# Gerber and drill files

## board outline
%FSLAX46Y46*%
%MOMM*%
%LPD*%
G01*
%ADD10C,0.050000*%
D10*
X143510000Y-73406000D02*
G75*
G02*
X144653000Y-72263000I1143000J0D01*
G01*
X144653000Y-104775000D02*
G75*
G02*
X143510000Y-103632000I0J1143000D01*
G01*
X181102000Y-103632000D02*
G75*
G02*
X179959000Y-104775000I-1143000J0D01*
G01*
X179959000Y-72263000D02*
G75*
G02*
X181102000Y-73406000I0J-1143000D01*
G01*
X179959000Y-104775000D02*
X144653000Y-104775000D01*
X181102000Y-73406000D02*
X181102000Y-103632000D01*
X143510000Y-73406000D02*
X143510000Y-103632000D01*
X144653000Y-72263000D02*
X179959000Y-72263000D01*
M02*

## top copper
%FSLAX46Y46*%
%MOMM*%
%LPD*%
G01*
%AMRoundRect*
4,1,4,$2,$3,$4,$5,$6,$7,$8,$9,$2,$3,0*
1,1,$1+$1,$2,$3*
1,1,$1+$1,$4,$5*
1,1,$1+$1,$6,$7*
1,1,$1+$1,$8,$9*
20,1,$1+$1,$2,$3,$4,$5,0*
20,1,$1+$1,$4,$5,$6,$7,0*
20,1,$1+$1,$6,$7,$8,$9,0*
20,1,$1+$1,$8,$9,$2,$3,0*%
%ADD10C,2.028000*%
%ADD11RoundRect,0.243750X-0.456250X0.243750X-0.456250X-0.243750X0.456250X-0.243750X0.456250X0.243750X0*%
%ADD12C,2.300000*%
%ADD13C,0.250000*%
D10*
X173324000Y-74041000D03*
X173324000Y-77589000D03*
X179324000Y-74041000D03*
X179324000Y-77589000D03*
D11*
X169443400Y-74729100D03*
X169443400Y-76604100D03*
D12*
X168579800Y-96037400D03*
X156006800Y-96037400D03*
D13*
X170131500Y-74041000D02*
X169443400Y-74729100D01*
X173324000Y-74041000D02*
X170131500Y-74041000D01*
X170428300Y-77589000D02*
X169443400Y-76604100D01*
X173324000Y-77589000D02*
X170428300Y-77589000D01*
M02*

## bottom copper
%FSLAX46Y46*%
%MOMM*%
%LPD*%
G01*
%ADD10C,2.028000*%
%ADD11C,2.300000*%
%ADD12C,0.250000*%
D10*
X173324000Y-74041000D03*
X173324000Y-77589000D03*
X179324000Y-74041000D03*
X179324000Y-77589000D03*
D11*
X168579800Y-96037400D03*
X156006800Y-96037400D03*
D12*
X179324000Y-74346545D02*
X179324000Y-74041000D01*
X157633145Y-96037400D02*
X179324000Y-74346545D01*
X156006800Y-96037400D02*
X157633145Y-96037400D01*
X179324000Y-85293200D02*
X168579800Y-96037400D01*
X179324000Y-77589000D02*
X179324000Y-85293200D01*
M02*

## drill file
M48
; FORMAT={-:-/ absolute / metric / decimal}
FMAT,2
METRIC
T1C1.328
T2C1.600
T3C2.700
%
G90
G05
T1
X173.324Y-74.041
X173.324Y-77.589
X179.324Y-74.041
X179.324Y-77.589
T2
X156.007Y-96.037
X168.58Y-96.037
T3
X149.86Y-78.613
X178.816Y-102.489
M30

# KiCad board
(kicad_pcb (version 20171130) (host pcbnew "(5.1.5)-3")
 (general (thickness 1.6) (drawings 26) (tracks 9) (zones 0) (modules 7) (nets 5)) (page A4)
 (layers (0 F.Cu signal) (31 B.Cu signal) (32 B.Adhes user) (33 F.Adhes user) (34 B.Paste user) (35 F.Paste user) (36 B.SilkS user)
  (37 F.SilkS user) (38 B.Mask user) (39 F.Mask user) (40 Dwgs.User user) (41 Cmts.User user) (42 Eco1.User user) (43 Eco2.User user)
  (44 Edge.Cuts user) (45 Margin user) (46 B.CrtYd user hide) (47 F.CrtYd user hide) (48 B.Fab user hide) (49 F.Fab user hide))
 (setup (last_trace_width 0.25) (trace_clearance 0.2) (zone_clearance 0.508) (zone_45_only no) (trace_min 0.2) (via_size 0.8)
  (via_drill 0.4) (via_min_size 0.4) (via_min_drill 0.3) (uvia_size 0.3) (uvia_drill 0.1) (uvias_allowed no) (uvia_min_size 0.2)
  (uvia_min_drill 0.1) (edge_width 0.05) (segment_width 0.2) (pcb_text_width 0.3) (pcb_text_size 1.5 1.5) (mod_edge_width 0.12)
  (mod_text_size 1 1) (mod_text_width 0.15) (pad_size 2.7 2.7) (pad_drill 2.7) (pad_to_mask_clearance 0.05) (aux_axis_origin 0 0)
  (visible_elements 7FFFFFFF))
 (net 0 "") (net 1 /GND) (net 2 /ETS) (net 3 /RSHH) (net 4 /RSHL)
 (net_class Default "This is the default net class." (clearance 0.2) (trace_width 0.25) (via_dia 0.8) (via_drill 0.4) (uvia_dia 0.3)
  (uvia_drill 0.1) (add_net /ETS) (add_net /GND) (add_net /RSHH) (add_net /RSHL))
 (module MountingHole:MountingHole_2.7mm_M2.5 (layer F.Cu) (at 178.816 102.489)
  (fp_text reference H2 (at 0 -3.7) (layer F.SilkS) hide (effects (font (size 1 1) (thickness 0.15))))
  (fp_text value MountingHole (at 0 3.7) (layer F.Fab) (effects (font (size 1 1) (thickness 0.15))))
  (pad 1 np_thru_hole circle (at 0 0) (size 2.7 2.7) (drill 2.7) (layers *.Cu *.Mask)))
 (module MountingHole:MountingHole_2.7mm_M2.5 (layer F.Cu) (at 149.86 78.613)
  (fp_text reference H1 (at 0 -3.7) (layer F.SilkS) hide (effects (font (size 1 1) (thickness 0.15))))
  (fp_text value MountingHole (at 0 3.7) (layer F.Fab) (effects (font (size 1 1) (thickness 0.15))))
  (pad "" np_thru_hole circle (at 0 0) (size 2.7 2.7) (drill 2.7) (layers *.Cu *.Mask)))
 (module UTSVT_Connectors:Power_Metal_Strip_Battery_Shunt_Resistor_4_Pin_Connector (layer F.Cu) (at 176.324 75.589)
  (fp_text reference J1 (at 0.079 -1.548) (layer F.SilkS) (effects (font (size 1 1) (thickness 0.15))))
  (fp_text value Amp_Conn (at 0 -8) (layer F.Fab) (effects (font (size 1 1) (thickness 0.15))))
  (pad 4 thru_hole circle (at -3 -1.548) (size 2.028 2.028) (drill 1.328) (layers *.Cu *.Mask) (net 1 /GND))
  (pad 1 thru_hole circle (at -3 2) (size 2.028 2.028) (drill 1.328) (layers *.Cu *.Mask) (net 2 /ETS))
  (pad 3 thru_hole circle (at 3 -1.548) (size 2.028 2.028) (drill 1.328) (layers *.Cu *.Mask) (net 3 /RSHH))
  (pad 2 thru_hole circle (at 3 2) (size 2.028 2.028) (drill 1.328) (layers *.Cu *.Mask) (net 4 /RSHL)))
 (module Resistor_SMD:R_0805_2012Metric (layer F.Cu) (at 169.4434 75.6666 270)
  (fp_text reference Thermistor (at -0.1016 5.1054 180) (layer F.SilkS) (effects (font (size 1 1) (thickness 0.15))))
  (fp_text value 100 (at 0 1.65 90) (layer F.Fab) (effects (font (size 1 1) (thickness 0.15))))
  (pad 1 smd roundrect (at -0.9375 0 270) (size 0.975 1.4) (layers F.Cu F.Paste F.Mask) (roundrect_rratio 0.25) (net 1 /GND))
  (pad 2 smd roundrect (at 0.9375 0 270) (size 0.975 1.4) (layers F.Cu F.Paste F.Mask) (roundrect_rratio 0.25) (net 2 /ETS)))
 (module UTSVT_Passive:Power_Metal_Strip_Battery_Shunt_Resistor (layer F.Cu) (at 162.2568 96.0374)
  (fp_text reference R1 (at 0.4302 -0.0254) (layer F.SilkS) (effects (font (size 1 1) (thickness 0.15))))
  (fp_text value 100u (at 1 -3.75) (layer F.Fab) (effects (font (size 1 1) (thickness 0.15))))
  (pad 2 thru_hole circle (at 6.323 0) (size 2.3 2.3) (drill 1.6) (layers *.Cu *.Mask) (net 4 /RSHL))
  (pad 1 thru_hole circle (at -6.25 0) (size 2.3 2.3) (drill 1.6) (layers *.Cu *.Mask) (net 3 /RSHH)))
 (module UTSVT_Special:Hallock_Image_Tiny (layer B.Cu) (at 163.322 84.709 180)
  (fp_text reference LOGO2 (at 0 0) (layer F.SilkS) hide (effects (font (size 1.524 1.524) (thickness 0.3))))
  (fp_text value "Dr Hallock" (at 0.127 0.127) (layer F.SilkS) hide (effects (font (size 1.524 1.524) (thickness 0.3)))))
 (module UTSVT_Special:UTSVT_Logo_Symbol (layer F.Cu) (at 162.179 84.582)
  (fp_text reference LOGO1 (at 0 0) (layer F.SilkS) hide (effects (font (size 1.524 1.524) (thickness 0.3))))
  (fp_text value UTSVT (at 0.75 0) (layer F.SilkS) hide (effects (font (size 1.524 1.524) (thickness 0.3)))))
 (gr_arc (start 144.653 73.406) (end 144.653 72.263) (angle -90) (layer Edge.Cuts) (width 0.05))
 (gr_arc (start 144.653 103.632) (end 143.51 103.632) (angle -90) (layer Edge.Cuts) (width 0.05))
 (gr_arc (start 179.959 103.632) (end 179.959 104.775) (angle -90) (layer Edge.Cuts) (width 0.05))
 (gr_arc (start 179.959 73.406) (end 181.102 73.406) (angle -90) (layer Edge.Cuts) (width 0.05))
 (gr_line (start 179.959 104.775) (end 144.653 104.775) (layer Edge.Cuts) (width 0.05))
 (gr_line (start 181.102 73.406) (end 181.102 103.632) (layer Edge.Cuts) (width 0.05))
 (gr_line (start 143.51 73.406) (end 143.51 103.632) (layer Edge.Cuts) (width 0.05))
 (gr_line (start 144.653 72.263) (end 179.959 72.263) (layer Edge.Cuts) (width 0.05))
 (segment (start 170.1315 74.041) (end 169.4434 74.7291) (width 0.25) (layer F.Cu) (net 1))
 (segment (start 173.324 74.041) (end 170.1315 74.041) (width 0.25) (layer F.Cu) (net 1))
 (segment (start 170.4283 77.589) (end 169.4434 76.6041) (width 0.25) (layer F.Cu) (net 2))
 (segment (start 173.324 77.589) (end 170.4283 77.589) (width 0.25) (layer F.Cu) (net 2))
 (segment (start 179.324 74.346545) (end 179.324 74.041) (width 0.25) (layer B.Cu) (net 3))
 (segment (start 157.633145 96.0374) (end 179.324 74.346545) (width 0.25) (layer B.Cu) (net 3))
 (segment (start 156.0068 96.0374) (end 157.633145 96.0374) (width 0.25) (layer B.Cu) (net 3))
 (segment (start 179.324 85.2932) (end 168.5798 96.0374) (width 0.25) (layer B.Cu) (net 4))
 (segment (start 179.324 77.589) (end 179.324 85.2932) (width 0.25) (layer B.Cu) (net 4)))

